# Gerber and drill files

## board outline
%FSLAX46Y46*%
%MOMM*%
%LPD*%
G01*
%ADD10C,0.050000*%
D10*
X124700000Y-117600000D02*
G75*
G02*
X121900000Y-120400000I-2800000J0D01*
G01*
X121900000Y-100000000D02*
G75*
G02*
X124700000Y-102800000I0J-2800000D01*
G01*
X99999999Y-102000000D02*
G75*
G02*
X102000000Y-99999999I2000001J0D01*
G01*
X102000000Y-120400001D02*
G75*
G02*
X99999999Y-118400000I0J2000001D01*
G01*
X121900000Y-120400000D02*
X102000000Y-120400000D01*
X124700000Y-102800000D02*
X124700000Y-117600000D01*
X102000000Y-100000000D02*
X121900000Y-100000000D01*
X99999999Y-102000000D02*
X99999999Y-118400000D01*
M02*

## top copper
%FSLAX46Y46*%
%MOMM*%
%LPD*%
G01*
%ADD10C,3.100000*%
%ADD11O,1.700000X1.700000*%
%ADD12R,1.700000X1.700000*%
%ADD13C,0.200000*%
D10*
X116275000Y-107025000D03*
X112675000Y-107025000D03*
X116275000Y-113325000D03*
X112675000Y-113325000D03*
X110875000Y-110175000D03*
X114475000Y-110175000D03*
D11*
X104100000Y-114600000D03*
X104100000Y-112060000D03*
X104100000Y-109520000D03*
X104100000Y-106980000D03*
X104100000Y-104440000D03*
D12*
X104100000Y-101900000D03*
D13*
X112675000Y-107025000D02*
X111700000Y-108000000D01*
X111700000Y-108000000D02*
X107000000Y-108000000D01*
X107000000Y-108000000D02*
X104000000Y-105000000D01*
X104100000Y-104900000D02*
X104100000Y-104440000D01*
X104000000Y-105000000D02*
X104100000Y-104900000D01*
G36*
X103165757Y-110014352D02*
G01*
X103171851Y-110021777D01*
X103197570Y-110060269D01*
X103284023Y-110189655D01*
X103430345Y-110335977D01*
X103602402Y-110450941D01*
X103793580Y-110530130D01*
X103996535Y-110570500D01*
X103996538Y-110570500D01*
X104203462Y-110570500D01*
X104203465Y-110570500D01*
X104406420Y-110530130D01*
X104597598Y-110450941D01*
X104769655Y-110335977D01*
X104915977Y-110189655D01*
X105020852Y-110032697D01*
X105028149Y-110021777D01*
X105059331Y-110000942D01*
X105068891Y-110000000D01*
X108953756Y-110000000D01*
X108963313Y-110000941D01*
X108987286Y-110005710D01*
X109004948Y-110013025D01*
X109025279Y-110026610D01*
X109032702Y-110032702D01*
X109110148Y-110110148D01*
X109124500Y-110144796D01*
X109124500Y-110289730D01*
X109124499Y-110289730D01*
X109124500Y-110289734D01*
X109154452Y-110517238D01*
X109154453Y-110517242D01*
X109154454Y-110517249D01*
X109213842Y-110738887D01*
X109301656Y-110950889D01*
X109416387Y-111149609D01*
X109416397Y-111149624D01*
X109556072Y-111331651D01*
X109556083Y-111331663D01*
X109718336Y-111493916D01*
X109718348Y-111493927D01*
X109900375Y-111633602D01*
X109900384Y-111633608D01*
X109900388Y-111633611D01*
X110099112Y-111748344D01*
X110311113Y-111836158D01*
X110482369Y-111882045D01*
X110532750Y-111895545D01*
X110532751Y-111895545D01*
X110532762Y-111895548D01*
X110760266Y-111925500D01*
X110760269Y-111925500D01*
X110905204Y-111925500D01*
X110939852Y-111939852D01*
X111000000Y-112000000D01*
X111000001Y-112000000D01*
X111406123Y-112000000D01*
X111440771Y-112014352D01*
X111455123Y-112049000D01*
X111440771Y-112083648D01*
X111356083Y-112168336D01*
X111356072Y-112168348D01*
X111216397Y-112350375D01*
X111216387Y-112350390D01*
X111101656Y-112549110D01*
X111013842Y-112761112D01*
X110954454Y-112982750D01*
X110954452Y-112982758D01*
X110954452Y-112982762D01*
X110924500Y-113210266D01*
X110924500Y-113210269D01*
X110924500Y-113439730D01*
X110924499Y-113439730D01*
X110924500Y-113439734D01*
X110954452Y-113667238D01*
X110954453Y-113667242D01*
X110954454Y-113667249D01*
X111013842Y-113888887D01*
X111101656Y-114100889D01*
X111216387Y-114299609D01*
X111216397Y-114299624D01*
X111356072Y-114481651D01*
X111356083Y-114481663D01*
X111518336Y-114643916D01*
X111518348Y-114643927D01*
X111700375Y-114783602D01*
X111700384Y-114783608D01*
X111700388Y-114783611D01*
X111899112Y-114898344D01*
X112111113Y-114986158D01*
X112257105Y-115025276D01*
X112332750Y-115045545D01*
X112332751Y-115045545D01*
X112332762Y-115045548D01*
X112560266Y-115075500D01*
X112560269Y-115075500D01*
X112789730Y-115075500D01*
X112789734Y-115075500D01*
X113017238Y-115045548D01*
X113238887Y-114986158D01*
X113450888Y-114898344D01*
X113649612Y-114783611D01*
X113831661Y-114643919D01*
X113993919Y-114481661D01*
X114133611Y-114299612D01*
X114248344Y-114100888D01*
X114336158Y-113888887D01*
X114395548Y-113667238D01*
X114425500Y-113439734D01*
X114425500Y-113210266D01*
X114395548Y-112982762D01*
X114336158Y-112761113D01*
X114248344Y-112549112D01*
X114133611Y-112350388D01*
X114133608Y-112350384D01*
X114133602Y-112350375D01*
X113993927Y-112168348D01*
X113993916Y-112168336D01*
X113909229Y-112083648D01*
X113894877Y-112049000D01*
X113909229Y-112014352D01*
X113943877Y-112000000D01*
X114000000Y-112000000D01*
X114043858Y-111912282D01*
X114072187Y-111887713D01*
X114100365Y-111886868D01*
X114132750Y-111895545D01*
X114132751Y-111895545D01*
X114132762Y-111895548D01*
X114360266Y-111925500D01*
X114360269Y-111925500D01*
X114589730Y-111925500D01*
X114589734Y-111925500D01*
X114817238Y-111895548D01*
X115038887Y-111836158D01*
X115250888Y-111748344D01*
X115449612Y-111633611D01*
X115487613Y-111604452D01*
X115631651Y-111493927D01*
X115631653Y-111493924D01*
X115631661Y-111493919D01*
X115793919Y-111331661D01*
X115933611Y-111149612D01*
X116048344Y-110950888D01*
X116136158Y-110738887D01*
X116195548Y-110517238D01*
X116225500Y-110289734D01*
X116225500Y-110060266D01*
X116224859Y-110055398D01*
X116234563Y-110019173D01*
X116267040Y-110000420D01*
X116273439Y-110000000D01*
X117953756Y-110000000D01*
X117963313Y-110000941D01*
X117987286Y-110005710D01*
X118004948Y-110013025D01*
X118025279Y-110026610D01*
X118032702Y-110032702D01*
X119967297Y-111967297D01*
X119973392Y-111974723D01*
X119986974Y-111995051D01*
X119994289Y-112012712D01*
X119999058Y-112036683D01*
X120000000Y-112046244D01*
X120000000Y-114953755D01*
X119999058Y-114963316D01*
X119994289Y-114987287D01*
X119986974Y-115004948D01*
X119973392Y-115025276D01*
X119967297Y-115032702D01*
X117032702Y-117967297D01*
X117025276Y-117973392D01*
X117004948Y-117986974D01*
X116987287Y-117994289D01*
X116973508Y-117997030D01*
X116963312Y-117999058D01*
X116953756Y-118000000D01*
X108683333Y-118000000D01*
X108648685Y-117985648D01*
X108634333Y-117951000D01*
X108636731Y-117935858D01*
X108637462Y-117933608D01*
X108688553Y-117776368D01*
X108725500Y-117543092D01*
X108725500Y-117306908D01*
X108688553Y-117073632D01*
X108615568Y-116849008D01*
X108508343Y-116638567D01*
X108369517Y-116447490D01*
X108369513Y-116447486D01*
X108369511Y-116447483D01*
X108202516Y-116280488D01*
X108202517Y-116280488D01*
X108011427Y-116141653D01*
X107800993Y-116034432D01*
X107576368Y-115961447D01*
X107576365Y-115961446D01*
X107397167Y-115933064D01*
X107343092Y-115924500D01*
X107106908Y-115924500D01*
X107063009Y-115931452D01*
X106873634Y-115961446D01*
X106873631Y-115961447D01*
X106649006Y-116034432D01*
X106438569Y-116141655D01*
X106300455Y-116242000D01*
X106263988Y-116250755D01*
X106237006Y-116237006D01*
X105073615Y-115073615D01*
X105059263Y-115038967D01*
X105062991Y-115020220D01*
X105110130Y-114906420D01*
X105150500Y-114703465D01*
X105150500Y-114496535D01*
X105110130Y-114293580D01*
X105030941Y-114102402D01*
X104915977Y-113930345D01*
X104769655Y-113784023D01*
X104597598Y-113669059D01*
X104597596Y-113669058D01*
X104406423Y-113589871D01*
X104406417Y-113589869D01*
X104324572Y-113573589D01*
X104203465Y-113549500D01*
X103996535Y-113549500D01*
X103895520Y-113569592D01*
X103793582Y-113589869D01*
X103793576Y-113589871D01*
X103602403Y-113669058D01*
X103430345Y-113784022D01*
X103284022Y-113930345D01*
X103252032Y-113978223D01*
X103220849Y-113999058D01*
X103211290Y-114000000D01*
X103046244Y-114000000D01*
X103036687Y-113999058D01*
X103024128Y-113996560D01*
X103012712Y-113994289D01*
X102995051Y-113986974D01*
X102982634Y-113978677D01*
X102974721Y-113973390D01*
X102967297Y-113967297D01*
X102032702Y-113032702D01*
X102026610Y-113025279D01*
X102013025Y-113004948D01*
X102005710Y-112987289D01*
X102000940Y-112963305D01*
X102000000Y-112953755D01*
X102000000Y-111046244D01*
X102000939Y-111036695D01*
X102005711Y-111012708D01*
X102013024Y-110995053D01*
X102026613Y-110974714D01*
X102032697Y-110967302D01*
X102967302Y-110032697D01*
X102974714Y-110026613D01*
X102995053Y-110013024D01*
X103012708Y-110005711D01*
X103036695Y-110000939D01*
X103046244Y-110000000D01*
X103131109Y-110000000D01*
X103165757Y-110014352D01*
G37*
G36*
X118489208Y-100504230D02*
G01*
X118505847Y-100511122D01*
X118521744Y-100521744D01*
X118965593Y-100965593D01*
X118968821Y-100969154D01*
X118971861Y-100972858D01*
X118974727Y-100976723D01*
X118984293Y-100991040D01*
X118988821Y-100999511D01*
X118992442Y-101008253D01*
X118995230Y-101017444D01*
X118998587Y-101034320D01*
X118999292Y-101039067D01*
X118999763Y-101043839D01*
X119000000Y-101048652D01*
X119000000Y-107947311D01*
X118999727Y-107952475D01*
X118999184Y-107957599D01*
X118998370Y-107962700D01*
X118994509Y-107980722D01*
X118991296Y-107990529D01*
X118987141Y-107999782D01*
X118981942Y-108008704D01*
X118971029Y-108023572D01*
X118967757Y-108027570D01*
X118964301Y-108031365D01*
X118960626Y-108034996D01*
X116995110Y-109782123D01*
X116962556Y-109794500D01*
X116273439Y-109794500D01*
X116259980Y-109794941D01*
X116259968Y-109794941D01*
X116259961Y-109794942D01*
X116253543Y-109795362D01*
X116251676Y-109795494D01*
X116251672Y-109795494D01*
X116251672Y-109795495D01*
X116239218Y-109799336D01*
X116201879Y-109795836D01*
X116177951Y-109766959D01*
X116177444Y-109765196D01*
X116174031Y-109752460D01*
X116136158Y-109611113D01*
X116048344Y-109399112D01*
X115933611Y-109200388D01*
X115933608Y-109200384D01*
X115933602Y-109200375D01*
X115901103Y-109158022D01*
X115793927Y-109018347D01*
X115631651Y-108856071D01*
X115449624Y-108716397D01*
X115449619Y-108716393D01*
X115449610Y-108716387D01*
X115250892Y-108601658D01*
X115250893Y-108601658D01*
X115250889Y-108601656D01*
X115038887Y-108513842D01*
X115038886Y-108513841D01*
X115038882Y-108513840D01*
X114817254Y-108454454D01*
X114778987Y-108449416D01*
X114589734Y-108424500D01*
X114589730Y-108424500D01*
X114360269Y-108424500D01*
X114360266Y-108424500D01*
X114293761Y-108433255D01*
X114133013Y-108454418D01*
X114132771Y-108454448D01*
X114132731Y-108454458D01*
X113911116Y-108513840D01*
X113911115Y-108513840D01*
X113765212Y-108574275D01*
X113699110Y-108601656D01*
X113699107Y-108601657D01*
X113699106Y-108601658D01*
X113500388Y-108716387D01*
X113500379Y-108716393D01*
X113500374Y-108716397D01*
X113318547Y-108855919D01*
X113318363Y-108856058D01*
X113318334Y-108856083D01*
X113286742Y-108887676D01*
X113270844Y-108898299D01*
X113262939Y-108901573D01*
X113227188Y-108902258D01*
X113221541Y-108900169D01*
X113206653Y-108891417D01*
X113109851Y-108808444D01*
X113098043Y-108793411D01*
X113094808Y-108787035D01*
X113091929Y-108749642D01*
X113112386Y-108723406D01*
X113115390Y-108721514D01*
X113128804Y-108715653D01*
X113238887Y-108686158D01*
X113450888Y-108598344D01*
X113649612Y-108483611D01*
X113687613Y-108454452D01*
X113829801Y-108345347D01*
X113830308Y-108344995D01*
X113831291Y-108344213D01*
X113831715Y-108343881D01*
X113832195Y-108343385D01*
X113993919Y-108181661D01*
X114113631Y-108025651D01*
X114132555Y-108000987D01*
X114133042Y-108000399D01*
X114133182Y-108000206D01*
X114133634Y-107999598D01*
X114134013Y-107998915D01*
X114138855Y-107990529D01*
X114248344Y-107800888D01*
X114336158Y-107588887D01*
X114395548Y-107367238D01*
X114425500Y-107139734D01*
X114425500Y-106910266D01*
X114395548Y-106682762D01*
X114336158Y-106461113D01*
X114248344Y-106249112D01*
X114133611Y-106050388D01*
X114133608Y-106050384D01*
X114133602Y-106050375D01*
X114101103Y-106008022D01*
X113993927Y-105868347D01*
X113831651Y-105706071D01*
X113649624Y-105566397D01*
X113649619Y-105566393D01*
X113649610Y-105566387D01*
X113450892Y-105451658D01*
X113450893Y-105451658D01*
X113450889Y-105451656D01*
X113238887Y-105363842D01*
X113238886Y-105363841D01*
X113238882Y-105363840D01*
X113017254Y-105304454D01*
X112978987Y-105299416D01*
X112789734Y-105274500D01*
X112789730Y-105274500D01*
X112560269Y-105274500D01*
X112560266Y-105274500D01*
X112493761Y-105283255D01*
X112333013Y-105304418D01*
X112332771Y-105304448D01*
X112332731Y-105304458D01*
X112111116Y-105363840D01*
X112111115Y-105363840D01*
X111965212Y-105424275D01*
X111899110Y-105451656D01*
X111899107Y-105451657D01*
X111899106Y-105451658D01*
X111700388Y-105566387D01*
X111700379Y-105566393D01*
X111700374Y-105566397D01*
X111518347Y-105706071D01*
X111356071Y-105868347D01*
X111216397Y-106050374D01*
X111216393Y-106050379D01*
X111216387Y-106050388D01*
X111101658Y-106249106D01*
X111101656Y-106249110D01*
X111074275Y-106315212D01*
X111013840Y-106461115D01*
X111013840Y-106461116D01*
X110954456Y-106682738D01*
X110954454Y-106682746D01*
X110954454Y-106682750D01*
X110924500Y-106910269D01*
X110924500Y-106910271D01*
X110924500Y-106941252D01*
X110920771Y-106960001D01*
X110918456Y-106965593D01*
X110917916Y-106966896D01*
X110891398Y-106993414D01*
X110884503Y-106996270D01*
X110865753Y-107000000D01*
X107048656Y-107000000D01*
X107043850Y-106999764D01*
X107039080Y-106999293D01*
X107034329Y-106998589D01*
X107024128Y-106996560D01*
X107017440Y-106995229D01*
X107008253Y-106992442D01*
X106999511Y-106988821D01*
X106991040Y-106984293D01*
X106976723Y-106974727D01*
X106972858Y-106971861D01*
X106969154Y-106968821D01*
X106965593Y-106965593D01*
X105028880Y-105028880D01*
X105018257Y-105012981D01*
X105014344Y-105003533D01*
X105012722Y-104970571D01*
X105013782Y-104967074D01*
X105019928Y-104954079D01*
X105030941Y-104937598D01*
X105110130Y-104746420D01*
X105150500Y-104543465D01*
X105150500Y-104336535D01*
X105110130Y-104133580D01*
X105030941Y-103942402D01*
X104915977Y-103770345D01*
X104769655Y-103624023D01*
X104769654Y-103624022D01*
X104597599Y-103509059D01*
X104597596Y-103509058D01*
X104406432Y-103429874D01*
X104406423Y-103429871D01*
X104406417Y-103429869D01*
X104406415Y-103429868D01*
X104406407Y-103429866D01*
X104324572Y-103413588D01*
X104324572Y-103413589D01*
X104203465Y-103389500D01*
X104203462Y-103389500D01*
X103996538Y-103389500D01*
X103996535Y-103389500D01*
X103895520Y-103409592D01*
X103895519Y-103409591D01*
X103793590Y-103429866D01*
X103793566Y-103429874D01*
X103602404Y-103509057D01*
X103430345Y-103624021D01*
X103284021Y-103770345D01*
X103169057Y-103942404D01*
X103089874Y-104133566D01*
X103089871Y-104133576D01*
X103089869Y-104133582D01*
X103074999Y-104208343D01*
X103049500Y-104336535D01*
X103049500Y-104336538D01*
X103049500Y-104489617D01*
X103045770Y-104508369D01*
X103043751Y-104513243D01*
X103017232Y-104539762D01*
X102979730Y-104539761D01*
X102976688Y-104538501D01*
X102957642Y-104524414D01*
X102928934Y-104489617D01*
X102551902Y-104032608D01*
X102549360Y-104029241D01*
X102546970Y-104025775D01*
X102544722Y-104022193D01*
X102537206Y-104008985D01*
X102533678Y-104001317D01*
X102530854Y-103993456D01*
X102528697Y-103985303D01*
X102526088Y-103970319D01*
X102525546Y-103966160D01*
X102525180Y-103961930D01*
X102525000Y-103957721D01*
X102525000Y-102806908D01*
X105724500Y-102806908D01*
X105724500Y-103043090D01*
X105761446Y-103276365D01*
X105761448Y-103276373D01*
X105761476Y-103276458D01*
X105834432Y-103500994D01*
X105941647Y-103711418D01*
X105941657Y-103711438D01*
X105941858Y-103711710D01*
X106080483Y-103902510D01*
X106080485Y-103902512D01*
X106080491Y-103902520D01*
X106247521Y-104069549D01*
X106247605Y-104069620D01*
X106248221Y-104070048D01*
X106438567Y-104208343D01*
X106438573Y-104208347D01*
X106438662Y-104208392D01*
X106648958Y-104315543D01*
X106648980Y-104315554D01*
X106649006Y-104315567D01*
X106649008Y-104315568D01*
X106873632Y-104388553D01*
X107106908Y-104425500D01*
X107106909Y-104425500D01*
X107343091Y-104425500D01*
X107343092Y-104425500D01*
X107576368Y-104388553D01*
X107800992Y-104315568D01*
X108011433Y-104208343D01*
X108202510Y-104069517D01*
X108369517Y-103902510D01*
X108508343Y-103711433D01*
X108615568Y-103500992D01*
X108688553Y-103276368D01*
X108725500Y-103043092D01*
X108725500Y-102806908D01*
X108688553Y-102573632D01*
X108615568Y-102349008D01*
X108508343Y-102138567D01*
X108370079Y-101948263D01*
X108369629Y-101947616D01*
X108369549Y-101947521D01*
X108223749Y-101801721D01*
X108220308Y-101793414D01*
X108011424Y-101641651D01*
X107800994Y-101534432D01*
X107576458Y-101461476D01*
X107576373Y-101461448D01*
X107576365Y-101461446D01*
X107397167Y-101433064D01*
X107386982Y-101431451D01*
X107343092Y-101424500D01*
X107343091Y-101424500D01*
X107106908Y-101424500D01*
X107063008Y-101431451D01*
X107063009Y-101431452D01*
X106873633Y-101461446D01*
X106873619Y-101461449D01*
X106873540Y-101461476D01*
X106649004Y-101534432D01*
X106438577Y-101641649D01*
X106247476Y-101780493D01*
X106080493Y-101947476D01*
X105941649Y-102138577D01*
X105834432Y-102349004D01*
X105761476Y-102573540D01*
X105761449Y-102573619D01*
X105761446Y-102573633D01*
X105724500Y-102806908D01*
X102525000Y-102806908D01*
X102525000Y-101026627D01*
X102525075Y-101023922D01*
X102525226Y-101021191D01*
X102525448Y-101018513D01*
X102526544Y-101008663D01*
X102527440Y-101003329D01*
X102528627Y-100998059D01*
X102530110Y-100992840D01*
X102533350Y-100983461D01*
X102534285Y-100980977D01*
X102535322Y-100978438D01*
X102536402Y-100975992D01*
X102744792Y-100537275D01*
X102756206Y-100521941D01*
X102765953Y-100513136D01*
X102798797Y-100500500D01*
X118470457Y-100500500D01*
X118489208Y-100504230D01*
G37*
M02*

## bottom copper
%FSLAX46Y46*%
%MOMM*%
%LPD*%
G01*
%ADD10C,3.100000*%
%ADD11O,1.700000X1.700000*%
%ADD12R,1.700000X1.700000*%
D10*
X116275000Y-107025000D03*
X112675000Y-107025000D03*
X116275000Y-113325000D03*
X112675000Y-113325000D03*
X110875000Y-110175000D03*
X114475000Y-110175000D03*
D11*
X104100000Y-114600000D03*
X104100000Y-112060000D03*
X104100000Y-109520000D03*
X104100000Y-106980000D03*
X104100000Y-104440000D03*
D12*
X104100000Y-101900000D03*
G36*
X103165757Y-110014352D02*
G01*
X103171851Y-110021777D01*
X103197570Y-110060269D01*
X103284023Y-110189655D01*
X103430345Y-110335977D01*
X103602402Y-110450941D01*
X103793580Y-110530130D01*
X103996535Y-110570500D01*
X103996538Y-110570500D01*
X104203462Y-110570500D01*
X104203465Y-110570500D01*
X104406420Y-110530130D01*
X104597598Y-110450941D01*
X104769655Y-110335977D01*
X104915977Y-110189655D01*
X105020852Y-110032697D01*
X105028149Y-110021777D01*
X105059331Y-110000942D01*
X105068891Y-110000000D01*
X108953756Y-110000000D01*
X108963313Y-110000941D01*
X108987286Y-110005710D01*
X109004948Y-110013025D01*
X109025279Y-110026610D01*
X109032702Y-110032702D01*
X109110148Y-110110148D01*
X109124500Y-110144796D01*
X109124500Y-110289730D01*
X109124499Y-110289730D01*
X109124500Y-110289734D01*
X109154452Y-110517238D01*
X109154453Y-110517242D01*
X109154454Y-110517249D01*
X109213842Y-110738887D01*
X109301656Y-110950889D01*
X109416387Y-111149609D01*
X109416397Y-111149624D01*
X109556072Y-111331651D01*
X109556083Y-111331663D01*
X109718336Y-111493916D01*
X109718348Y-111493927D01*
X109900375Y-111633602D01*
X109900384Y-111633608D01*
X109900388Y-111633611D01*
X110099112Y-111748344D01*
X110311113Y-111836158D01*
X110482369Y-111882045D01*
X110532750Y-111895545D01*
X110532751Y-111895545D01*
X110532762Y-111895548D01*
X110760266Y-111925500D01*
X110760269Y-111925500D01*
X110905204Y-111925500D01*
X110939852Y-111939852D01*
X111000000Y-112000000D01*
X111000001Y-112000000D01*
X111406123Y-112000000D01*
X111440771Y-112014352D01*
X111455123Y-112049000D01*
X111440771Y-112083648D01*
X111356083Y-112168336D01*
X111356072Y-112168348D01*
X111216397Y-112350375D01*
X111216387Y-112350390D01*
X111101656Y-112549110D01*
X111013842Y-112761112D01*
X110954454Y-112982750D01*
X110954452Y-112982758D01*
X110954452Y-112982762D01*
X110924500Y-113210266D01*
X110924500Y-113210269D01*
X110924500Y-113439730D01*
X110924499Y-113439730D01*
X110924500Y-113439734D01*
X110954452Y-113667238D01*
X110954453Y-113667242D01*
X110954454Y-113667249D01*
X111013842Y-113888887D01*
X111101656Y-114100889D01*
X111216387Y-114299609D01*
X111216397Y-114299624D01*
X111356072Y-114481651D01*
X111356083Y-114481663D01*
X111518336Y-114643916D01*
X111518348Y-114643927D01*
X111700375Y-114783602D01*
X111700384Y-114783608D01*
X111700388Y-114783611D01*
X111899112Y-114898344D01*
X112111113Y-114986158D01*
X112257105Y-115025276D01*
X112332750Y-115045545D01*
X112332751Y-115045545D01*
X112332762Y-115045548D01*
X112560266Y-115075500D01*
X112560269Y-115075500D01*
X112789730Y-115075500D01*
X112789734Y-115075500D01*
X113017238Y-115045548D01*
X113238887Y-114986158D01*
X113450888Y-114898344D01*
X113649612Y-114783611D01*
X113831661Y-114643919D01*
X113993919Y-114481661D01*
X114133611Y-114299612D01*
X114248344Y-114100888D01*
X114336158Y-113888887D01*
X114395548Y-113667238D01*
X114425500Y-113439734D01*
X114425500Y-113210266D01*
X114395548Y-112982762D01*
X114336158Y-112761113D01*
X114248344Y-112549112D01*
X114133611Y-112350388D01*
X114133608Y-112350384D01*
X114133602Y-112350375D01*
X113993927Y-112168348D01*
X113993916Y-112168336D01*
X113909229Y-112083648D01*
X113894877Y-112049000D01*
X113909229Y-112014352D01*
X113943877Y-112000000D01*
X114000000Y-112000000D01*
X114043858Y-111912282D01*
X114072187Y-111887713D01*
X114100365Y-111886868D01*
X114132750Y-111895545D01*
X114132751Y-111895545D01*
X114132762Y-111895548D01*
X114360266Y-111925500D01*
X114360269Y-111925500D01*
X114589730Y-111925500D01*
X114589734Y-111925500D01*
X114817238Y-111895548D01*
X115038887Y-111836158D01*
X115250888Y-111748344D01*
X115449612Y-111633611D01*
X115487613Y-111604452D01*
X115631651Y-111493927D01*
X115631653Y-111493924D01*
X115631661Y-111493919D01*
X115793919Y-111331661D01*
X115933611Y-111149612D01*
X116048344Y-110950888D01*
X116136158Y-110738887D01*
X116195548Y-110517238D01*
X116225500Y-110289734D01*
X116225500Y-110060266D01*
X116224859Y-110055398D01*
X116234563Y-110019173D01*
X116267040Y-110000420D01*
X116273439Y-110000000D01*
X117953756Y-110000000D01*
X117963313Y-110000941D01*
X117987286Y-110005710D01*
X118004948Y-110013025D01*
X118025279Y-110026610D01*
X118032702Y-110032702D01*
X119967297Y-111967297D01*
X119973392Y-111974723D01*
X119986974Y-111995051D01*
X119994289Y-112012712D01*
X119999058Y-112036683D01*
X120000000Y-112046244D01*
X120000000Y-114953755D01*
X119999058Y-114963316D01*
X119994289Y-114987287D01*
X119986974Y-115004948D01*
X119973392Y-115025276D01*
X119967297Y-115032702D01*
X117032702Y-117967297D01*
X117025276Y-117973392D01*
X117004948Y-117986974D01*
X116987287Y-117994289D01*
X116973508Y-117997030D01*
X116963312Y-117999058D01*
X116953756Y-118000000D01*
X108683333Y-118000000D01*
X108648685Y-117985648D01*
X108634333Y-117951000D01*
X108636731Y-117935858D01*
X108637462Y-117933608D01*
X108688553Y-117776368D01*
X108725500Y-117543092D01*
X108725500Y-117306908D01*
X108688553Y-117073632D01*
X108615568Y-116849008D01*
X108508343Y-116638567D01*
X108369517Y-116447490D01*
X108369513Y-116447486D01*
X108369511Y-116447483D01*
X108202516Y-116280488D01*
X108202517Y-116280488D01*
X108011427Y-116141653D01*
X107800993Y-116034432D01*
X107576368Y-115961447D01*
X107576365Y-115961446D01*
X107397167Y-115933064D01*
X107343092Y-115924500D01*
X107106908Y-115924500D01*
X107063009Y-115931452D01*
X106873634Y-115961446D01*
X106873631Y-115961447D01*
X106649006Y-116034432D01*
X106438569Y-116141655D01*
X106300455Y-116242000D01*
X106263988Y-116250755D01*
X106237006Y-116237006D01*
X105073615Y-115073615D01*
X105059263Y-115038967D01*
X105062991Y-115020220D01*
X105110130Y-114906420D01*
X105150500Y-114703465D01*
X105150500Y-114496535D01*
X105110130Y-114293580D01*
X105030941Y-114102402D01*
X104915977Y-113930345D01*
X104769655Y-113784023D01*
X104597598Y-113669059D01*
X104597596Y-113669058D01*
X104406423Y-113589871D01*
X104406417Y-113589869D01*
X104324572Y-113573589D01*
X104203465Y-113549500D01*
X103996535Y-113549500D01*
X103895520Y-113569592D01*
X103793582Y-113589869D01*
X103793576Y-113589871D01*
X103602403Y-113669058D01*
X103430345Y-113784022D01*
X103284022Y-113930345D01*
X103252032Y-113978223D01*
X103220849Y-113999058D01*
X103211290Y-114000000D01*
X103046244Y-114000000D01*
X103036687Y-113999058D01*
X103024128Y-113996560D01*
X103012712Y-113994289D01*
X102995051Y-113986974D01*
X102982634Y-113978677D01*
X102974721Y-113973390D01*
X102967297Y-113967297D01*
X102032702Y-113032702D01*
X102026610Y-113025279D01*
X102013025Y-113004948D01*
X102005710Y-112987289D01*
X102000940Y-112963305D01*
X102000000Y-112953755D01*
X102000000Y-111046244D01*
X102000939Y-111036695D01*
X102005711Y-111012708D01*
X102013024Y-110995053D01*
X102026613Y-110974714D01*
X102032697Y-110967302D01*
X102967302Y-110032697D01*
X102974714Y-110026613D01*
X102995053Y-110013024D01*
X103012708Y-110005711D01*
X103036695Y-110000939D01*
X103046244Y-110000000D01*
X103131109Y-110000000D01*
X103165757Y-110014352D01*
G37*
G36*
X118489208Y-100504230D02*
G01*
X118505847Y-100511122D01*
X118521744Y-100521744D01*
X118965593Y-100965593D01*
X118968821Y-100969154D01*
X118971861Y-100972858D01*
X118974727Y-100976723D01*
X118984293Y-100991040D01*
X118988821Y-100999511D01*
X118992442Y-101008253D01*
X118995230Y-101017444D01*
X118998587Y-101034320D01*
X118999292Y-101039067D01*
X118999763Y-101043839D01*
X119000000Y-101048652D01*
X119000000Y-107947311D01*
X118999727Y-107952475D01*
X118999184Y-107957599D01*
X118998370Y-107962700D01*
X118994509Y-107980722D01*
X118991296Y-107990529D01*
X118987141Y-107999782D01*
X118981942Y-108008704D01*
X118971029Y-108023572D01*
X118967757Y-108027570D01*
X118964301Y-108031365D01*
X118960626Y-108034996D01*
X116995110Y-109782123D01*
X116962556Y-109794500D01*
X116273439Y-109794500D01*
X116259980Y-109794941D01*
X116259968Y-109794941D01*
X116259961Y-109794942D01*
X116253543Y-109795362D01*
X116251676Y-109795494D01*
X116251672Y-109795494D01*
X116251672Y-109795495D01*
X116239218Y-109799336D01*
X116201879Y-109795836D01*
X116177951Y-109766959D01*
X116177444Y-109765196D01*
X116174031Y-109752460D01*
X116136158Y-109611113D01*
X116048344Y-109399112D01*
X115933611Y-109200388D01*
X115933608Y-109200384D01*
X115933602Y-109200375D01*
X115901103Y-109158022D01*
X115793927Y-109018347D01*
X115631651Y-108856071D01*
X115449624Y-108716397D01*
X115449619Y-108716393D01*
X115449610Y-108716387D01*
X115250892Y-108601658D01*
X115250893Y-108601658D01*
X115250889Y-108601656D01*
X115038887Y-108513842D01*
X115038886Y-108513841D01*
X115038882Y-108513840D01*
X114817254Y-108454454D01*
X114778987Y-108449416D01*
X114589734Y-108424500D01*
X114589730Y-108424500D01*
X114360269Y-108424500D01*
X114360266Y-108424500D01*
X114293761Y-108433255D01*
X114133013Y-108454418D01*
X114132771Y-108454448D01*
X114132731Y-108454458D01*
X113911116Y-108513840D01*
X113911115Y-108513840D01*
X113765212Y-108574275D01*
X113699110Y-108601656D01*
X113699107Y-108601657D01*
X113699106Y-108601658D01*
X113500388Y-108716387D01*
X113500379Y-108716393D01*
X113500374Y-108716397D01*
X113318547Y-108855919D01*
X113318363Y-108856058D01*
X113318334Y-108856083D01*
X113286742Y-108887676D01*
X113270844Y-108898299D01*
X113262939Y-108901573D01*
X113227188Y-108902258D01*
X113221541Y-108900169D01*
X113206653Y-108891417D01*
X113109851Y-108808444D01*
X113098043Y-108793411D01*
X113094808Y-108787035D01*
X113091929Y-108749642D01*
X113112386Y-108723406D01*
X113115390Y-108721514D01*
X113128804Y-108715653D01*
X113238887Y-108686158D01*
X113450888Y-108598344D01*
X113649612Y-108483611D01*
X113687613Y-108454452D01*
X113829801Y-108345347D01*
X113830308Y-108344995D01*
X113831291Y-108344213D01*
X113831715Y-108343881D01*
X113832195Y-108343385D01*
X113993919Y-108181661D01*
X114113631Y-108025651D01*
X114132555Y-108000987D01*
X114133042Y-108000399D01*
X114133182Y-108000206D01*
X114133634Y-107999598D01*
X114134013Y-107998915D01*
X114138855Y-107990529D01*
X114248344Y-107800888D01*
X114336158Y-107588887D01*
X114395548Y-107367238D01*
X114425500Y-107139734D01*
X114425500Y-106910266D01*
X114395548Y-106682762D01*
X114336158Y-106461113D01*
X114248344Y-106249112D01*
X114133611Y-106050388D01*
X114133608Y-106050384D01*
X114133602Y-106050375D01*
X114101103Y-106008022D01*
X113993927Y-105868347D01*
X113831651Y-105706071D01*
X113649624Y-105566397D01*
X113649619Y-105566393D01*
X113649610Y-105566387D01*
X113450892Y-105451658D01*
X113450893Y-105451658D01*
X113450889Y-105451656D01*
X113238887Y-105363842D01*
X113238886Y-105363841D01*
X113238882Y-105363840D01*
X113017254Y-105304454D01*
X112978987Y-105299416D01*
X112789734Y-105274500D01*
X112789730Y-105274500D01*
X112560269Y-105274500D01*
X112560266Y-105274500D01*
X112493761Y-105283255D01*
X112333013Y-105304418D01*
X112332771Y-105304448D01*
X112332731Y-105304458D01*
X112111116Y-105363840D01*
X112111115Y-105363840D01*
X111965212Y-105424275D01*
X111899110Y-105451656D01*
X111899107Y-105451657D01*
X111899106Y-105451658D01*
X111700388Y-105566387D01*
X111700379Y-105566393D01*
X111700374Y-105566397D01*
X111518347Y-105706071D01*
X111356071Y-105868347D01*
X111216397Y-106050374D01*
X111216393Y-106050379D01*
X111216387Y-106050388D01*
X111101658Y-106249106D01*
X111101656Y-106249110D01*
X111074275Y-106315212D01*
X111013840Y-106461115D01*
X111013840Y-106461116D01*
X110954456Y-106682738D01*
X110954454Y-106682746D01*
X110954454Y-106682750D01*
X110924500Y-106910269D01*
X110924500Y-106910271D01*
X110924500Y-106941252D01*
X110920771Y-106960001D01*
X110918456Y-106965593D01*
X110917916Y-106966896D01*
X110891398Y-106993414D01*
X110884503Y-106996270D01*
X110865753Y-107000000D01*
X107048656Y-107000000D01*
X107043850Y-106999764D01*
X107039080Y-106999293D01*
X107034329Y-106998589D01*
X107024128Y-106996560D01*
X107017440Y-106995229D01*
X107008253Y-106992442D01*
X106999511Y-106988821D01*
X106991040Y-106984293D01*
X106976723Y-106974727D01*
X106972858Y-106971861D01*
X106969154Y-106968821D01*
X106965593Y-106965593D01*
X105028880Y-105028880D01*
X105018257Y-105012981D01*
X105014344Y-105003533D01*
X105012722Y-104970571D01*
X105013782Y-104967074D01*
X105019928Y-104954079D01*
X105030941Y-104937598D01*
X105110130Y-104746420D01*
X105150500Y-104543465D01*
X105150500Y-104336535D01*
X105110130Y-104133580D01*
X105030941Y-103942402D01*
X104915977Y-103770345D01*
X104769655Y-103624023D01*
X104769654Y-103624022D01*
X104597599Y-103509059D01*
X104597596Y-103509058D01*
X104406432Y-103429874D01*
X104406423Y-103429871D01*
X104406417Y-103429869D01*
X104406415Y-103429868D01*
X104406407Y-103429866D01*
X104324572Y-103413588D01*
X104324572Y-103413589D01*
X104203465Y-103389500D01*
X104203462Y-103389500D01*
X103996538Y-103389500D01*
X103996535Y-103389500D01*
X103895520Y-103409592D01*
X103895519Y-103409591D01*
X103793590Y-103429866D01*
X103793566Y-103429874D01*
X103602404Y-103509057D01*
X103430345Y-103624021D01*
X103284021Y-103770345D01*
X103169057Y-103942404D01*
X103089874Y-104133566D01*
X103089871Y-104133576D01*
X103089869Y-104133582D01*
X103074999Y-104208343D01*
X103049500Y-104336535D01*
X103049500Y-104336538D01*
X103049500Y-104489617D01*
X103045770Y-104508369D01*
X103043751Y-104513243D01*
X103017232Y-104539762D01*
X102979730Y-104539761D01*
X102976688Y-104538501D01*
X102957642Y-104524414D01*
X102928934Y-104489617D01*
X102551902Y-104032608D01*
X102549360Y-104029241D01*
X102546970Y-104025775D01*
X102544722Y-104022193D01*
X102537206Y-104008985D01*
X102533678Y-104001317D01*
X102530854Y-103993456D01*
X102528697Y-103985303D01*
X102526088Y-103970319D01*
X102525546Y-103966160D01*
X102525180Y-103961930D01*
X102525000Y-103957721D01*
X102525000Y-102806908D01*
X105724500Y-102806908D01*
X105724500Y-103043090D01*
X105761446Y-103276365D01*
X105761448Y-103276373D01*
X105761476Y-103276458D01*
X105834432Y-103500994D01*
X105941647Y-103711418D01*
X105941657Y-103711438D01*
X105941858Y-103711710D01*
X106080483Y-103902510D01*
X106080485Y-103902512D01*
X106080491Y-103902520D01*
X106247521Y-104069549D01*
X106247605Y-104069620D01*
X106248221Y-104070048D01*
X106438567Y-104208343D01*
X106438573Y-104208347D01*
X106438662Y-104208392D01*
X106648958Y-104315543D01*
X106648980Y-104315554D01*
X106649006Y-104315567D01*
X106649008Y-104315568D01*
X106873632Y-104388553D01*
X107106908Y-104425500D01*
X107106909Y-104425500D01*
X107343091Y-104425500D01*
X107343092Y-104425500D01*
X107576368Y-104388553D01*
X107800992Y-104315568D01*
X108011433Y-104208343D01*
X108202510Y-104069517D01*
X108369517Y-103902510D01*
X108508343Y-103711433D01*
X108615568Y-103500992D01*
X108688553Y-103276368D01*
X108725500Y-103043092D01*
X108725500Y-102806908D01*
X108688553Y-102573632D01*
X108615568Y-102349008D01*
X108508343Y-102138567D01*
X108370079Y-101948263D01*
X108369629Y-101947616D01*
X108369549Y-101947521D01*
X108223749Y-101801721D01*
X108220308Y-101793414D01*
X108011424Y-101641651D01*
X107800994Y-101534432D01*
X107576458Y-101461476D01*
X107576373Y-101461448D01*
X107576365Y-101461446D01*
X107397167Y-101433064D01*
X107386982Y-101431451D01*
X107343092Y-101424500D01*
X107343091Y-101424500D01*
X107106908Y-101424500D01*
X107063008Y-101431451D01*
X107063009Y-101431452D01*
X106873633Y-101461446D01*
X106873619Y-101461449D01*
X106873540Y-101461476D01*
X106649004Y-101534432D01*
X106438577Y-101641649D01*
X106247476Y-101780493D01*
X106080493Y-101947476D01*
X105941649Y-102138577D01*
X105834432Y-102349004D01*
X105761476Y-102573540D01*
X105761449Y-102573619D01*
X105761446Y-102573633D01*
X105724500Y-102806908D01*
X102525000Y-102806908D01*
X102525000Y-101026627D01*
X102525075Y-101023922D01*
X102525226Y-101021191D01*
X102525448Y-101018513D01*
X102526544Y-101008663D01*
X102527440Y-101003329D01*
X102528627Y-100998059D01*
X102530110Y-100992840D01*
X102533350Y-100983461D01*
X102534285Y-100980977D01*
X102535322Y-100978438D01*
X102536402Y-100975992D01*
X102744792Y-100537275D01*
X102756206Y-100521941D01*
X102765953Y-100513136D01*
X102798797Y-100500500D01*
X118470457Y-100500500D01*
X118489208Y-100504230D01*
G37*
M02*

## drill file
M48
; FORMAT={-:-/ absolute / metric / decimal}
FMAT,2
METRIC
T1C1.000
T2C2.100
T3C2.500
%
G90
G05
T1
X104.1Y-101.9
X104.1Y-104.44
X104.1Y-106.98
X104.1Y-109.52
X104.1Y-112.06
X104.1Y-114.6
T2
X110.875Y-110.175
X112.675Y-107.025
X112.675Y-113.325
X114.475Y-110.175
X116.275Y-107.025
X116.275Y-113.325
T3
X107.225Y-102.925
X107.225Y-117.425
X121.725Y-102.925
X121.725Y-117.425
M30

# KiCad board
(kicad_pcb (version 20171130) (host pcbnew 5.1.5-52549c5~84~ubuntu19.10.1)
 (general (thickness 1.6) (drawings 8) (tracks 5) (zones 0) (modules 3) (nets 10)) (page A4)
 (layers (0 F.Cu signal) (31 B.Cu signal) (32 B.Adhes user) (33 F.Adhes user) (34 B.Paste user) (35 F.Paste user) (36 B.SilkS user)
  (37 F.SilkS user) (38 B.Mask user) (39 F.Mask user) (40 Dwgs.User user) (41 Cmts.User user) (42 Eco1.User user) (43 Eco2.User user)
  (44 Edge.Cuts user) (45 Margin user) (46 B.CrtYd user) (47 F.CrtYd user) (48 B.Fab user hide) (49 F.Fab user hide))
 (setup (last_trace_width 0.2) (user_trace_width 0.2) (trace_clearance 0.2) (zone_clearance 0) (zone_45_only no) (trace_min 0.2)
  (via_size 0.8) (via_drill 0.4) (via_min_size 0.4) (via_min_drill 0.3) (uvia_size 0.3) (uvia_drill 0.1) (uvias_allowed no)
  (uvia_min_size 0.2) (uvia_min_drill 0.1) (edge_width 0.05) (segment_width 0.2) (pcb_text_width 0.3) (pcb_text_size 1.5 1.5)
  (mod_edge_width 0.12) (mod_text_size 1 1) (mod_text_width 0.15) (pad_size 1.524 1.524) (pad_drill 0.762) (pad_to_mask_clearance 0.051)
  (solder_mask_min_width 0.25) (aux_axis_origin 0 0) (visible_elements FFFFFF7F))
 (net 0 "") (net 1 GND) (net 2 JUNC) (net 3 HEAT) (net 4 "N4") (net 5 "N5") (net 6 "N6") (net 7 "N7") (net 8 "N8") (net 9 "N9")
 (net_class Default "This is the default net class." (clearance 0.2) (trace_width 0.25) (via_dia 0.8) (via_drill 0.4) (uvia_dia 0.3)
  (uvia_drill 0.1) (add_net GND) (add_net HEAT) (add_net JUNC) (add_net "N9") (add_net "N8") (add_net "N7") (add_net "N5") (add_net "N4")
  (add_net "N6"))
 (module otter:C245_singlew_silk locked (layer F.Cu) (at 101.5 110.2 270)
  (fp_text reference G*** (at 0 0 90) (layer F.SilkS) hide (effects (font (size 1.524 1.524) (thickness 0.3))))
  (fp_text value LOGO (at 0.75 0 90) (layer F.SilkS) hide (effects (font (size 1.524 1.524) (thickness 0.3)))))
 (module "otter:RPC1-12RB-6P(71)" (layer F.Cu) (at 114.475 110.175 180)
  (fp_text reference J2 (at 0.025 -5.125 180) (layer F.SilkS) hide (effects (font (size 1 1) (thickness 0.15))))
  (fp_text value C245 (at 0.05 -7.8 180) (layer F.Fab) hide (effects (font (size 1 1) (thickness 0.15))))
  (pad "" np_thru_hole circle (at -7.25 -7.25 180) (size 2.5 2.5) (drill 2.5) (layers *.Cu *.Mask))
  (pad "" np_thru_hole circle (at -7.25 7.25 180) (size 2.5 2.5) (drill 2.5) (layers *.Cu *.Mask))
  (pad "" np_thru_hole circle (at 7.25 7.25 180) (size 2.5 2.5) (drill 2.5) (layers *.Cu *.Mask))
  (pad "" np_thru_hole circle (at 7.25 -7.25 180) (size 2.5 2.5) (drill 2.5) (layers *.Cu *.Mask))
  (pad 1 thru_hole circle (at -1.8 3.15 180) (size 3.1 3.1) (drill 2.1) (layers *.Cu *.Mask) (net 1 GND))
  (pad 2 thru_hole circle (at 1.8 3.15 180) (size 3.1 3.1) (drill 2.1) (layers *.Cu *.Mask) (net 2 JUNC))
  (pad 5 thru_hole circle (at -1.8 -3.15 180) (size 3.1 3.1) (drill 2.1) (layers *.Cu *.Mask) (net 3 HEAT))
  (pad 4 thru_hole circle (at 1.8 -3.15 180) (size 3.1 3.1) (drill 2.1) (layers *.Cu *.Mask) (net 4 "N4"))
  (pad 3 thru_hole circle (at 3.6 0 180) (size 3.1 3.1) (drill 2.1) (layers *.Cu *.Mask) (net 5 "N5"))
  (pad 6 thru_hole circle (at 0 0 180) (size 3.1 3.1) (drill 2.1) (layers *.Cu *.Mask) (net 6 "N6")))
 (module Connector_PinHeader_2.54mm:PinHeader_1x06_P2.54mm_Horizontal (layer B.Cu) (at 104.1 101.9 180)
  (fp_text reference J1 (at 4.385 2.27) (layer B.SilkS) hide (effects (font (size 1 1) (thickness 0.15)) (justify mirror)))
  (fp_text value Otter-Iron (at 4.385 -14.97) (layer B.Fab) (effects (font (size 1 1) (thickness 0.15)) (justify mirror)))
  (pad 6 thru_hole oval (at 0 -12.7 180) (size 1.7 1.7) (drill 1) (layers *.Cu *.Mask) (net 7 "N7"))
  (pad 5 thru_hole oval (at 0 -10.16 180) (size 1.7 1.7) (drill 1) (layers *.Cu *.Mask) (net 3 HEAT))
  (pad 4 thru_hole oval (at 0 -7.62 180) (size 1.7 1.7) (drill 1) (layers *.Cu *.Mask) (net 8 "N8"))
  (pad 3 thru_hole oval (at 0 -5.08 180) (size 1.7 1.7) (drill 1) (layers *.Cu *.Mask) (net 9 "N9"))
  (pad 2 thru_hole oval (at 0 -2.54 180) (size 1.7 1.7) (drill 1) (layers *.Cu *.Mask) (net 2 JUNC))
  (pad 1 thru_hole rect (at 0 0 180) (size 1.7 1.7) (drill 1) (layers *.Cu *.Mask) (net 1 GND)))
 (gr_arc (start 121.9 117.6) (end 121.9 120.4) (angle -90) (layer Edge.Cuts) (width 0.05))
 (gr_arc (start 121.9 102.8) (end 124.7 102.8) (angle -90) (layer Edge.Cuts) (width 0.05))
 (gr_arc (start 102 102) (end 102 99.999999) (angle -90) (layer Edge.Cuts) (width 0.05))
 (gr_arc (start 102 118.4) (end 99.999999 118.4) (angle -90) (layer Edge.Cuts) (width 0.05))
 (gr_line (start 121.9 120.4) (end 102 120.4) (layer Edge.Cuts) (width 0.05))
 (gr_line (start 124.7 102.8) (end 124.7 117.6) (layer Edge.Cuts) (width 0.05))
 (gr_line (start 102 100) (end 121.9 100) (layer Edge.Cuts) (width 0.05))
 (gr_line (start 99.999999 102) (end 99.999999 118.4) (layer Edge.Cuts) (width 0.05))
 (segment (start 112.675 107.025) (end 111.7 108) (width 0.2) (layer F.Cu) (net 2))
 (segment (start 111.7 108) (end 107 108) (width 0.2) (layer F.Cu) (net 2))
 (segment (start 107 108) (end 104 105) (width 0.2) (layer F.Cu) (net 2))
 (segment (start 104.1 104.9) (end 104.1 104.44) (width 0.2) (layer F.Cu) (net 2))
 (segment (start 104 105) (end 104.1 104.9) (width 0.2) (layer F.Cu) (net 2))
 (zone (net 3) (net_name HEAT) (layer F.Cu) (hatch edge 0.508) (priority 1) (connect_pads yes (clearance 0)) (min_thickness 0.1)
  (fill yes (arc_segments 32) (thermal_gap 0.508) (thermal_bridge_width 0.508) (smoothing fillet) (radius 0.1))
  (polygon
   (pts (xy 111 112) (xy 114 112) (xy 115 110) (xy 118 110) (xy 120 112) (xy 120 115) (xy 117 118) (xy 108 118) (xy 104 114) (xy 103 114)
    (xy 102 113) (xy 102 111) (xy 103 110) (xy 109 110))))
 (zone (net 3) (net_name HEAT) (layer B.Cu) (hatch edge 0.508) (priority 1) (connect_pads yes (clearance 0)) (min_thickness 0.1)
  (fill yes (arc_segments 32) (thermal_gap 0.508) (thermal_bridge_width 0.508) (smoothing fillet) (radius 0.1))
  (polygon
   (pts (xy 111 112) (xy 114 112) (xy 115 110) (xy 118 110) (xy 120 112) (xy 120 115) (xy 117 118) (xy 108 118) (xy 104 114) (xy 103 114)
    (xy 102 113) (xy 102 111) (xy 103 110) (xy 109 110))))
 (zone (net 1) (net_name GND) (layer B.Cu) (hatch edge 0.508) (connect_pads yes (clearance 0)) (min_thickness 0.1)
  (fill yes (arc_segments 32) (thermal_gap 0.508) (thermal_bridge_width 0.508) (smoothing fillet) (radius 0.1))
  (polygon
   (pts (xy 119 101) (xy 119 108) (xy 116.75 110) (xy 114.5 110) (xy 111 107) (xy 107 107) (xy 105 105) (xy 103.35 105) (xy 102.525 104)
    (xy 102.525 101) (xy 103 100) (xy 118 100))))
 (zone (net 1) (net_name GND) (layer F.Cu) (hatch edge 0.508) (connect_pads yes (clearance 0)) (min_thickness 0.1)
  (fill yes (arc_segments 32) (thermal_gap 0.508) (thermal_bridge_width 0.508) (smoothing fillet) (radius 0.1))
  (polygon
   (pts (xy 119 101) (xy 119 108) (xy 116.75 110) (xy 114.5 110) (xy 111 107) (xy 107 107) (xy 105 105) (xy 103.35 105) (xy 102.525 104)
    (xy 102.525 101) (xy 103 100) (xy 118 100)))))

